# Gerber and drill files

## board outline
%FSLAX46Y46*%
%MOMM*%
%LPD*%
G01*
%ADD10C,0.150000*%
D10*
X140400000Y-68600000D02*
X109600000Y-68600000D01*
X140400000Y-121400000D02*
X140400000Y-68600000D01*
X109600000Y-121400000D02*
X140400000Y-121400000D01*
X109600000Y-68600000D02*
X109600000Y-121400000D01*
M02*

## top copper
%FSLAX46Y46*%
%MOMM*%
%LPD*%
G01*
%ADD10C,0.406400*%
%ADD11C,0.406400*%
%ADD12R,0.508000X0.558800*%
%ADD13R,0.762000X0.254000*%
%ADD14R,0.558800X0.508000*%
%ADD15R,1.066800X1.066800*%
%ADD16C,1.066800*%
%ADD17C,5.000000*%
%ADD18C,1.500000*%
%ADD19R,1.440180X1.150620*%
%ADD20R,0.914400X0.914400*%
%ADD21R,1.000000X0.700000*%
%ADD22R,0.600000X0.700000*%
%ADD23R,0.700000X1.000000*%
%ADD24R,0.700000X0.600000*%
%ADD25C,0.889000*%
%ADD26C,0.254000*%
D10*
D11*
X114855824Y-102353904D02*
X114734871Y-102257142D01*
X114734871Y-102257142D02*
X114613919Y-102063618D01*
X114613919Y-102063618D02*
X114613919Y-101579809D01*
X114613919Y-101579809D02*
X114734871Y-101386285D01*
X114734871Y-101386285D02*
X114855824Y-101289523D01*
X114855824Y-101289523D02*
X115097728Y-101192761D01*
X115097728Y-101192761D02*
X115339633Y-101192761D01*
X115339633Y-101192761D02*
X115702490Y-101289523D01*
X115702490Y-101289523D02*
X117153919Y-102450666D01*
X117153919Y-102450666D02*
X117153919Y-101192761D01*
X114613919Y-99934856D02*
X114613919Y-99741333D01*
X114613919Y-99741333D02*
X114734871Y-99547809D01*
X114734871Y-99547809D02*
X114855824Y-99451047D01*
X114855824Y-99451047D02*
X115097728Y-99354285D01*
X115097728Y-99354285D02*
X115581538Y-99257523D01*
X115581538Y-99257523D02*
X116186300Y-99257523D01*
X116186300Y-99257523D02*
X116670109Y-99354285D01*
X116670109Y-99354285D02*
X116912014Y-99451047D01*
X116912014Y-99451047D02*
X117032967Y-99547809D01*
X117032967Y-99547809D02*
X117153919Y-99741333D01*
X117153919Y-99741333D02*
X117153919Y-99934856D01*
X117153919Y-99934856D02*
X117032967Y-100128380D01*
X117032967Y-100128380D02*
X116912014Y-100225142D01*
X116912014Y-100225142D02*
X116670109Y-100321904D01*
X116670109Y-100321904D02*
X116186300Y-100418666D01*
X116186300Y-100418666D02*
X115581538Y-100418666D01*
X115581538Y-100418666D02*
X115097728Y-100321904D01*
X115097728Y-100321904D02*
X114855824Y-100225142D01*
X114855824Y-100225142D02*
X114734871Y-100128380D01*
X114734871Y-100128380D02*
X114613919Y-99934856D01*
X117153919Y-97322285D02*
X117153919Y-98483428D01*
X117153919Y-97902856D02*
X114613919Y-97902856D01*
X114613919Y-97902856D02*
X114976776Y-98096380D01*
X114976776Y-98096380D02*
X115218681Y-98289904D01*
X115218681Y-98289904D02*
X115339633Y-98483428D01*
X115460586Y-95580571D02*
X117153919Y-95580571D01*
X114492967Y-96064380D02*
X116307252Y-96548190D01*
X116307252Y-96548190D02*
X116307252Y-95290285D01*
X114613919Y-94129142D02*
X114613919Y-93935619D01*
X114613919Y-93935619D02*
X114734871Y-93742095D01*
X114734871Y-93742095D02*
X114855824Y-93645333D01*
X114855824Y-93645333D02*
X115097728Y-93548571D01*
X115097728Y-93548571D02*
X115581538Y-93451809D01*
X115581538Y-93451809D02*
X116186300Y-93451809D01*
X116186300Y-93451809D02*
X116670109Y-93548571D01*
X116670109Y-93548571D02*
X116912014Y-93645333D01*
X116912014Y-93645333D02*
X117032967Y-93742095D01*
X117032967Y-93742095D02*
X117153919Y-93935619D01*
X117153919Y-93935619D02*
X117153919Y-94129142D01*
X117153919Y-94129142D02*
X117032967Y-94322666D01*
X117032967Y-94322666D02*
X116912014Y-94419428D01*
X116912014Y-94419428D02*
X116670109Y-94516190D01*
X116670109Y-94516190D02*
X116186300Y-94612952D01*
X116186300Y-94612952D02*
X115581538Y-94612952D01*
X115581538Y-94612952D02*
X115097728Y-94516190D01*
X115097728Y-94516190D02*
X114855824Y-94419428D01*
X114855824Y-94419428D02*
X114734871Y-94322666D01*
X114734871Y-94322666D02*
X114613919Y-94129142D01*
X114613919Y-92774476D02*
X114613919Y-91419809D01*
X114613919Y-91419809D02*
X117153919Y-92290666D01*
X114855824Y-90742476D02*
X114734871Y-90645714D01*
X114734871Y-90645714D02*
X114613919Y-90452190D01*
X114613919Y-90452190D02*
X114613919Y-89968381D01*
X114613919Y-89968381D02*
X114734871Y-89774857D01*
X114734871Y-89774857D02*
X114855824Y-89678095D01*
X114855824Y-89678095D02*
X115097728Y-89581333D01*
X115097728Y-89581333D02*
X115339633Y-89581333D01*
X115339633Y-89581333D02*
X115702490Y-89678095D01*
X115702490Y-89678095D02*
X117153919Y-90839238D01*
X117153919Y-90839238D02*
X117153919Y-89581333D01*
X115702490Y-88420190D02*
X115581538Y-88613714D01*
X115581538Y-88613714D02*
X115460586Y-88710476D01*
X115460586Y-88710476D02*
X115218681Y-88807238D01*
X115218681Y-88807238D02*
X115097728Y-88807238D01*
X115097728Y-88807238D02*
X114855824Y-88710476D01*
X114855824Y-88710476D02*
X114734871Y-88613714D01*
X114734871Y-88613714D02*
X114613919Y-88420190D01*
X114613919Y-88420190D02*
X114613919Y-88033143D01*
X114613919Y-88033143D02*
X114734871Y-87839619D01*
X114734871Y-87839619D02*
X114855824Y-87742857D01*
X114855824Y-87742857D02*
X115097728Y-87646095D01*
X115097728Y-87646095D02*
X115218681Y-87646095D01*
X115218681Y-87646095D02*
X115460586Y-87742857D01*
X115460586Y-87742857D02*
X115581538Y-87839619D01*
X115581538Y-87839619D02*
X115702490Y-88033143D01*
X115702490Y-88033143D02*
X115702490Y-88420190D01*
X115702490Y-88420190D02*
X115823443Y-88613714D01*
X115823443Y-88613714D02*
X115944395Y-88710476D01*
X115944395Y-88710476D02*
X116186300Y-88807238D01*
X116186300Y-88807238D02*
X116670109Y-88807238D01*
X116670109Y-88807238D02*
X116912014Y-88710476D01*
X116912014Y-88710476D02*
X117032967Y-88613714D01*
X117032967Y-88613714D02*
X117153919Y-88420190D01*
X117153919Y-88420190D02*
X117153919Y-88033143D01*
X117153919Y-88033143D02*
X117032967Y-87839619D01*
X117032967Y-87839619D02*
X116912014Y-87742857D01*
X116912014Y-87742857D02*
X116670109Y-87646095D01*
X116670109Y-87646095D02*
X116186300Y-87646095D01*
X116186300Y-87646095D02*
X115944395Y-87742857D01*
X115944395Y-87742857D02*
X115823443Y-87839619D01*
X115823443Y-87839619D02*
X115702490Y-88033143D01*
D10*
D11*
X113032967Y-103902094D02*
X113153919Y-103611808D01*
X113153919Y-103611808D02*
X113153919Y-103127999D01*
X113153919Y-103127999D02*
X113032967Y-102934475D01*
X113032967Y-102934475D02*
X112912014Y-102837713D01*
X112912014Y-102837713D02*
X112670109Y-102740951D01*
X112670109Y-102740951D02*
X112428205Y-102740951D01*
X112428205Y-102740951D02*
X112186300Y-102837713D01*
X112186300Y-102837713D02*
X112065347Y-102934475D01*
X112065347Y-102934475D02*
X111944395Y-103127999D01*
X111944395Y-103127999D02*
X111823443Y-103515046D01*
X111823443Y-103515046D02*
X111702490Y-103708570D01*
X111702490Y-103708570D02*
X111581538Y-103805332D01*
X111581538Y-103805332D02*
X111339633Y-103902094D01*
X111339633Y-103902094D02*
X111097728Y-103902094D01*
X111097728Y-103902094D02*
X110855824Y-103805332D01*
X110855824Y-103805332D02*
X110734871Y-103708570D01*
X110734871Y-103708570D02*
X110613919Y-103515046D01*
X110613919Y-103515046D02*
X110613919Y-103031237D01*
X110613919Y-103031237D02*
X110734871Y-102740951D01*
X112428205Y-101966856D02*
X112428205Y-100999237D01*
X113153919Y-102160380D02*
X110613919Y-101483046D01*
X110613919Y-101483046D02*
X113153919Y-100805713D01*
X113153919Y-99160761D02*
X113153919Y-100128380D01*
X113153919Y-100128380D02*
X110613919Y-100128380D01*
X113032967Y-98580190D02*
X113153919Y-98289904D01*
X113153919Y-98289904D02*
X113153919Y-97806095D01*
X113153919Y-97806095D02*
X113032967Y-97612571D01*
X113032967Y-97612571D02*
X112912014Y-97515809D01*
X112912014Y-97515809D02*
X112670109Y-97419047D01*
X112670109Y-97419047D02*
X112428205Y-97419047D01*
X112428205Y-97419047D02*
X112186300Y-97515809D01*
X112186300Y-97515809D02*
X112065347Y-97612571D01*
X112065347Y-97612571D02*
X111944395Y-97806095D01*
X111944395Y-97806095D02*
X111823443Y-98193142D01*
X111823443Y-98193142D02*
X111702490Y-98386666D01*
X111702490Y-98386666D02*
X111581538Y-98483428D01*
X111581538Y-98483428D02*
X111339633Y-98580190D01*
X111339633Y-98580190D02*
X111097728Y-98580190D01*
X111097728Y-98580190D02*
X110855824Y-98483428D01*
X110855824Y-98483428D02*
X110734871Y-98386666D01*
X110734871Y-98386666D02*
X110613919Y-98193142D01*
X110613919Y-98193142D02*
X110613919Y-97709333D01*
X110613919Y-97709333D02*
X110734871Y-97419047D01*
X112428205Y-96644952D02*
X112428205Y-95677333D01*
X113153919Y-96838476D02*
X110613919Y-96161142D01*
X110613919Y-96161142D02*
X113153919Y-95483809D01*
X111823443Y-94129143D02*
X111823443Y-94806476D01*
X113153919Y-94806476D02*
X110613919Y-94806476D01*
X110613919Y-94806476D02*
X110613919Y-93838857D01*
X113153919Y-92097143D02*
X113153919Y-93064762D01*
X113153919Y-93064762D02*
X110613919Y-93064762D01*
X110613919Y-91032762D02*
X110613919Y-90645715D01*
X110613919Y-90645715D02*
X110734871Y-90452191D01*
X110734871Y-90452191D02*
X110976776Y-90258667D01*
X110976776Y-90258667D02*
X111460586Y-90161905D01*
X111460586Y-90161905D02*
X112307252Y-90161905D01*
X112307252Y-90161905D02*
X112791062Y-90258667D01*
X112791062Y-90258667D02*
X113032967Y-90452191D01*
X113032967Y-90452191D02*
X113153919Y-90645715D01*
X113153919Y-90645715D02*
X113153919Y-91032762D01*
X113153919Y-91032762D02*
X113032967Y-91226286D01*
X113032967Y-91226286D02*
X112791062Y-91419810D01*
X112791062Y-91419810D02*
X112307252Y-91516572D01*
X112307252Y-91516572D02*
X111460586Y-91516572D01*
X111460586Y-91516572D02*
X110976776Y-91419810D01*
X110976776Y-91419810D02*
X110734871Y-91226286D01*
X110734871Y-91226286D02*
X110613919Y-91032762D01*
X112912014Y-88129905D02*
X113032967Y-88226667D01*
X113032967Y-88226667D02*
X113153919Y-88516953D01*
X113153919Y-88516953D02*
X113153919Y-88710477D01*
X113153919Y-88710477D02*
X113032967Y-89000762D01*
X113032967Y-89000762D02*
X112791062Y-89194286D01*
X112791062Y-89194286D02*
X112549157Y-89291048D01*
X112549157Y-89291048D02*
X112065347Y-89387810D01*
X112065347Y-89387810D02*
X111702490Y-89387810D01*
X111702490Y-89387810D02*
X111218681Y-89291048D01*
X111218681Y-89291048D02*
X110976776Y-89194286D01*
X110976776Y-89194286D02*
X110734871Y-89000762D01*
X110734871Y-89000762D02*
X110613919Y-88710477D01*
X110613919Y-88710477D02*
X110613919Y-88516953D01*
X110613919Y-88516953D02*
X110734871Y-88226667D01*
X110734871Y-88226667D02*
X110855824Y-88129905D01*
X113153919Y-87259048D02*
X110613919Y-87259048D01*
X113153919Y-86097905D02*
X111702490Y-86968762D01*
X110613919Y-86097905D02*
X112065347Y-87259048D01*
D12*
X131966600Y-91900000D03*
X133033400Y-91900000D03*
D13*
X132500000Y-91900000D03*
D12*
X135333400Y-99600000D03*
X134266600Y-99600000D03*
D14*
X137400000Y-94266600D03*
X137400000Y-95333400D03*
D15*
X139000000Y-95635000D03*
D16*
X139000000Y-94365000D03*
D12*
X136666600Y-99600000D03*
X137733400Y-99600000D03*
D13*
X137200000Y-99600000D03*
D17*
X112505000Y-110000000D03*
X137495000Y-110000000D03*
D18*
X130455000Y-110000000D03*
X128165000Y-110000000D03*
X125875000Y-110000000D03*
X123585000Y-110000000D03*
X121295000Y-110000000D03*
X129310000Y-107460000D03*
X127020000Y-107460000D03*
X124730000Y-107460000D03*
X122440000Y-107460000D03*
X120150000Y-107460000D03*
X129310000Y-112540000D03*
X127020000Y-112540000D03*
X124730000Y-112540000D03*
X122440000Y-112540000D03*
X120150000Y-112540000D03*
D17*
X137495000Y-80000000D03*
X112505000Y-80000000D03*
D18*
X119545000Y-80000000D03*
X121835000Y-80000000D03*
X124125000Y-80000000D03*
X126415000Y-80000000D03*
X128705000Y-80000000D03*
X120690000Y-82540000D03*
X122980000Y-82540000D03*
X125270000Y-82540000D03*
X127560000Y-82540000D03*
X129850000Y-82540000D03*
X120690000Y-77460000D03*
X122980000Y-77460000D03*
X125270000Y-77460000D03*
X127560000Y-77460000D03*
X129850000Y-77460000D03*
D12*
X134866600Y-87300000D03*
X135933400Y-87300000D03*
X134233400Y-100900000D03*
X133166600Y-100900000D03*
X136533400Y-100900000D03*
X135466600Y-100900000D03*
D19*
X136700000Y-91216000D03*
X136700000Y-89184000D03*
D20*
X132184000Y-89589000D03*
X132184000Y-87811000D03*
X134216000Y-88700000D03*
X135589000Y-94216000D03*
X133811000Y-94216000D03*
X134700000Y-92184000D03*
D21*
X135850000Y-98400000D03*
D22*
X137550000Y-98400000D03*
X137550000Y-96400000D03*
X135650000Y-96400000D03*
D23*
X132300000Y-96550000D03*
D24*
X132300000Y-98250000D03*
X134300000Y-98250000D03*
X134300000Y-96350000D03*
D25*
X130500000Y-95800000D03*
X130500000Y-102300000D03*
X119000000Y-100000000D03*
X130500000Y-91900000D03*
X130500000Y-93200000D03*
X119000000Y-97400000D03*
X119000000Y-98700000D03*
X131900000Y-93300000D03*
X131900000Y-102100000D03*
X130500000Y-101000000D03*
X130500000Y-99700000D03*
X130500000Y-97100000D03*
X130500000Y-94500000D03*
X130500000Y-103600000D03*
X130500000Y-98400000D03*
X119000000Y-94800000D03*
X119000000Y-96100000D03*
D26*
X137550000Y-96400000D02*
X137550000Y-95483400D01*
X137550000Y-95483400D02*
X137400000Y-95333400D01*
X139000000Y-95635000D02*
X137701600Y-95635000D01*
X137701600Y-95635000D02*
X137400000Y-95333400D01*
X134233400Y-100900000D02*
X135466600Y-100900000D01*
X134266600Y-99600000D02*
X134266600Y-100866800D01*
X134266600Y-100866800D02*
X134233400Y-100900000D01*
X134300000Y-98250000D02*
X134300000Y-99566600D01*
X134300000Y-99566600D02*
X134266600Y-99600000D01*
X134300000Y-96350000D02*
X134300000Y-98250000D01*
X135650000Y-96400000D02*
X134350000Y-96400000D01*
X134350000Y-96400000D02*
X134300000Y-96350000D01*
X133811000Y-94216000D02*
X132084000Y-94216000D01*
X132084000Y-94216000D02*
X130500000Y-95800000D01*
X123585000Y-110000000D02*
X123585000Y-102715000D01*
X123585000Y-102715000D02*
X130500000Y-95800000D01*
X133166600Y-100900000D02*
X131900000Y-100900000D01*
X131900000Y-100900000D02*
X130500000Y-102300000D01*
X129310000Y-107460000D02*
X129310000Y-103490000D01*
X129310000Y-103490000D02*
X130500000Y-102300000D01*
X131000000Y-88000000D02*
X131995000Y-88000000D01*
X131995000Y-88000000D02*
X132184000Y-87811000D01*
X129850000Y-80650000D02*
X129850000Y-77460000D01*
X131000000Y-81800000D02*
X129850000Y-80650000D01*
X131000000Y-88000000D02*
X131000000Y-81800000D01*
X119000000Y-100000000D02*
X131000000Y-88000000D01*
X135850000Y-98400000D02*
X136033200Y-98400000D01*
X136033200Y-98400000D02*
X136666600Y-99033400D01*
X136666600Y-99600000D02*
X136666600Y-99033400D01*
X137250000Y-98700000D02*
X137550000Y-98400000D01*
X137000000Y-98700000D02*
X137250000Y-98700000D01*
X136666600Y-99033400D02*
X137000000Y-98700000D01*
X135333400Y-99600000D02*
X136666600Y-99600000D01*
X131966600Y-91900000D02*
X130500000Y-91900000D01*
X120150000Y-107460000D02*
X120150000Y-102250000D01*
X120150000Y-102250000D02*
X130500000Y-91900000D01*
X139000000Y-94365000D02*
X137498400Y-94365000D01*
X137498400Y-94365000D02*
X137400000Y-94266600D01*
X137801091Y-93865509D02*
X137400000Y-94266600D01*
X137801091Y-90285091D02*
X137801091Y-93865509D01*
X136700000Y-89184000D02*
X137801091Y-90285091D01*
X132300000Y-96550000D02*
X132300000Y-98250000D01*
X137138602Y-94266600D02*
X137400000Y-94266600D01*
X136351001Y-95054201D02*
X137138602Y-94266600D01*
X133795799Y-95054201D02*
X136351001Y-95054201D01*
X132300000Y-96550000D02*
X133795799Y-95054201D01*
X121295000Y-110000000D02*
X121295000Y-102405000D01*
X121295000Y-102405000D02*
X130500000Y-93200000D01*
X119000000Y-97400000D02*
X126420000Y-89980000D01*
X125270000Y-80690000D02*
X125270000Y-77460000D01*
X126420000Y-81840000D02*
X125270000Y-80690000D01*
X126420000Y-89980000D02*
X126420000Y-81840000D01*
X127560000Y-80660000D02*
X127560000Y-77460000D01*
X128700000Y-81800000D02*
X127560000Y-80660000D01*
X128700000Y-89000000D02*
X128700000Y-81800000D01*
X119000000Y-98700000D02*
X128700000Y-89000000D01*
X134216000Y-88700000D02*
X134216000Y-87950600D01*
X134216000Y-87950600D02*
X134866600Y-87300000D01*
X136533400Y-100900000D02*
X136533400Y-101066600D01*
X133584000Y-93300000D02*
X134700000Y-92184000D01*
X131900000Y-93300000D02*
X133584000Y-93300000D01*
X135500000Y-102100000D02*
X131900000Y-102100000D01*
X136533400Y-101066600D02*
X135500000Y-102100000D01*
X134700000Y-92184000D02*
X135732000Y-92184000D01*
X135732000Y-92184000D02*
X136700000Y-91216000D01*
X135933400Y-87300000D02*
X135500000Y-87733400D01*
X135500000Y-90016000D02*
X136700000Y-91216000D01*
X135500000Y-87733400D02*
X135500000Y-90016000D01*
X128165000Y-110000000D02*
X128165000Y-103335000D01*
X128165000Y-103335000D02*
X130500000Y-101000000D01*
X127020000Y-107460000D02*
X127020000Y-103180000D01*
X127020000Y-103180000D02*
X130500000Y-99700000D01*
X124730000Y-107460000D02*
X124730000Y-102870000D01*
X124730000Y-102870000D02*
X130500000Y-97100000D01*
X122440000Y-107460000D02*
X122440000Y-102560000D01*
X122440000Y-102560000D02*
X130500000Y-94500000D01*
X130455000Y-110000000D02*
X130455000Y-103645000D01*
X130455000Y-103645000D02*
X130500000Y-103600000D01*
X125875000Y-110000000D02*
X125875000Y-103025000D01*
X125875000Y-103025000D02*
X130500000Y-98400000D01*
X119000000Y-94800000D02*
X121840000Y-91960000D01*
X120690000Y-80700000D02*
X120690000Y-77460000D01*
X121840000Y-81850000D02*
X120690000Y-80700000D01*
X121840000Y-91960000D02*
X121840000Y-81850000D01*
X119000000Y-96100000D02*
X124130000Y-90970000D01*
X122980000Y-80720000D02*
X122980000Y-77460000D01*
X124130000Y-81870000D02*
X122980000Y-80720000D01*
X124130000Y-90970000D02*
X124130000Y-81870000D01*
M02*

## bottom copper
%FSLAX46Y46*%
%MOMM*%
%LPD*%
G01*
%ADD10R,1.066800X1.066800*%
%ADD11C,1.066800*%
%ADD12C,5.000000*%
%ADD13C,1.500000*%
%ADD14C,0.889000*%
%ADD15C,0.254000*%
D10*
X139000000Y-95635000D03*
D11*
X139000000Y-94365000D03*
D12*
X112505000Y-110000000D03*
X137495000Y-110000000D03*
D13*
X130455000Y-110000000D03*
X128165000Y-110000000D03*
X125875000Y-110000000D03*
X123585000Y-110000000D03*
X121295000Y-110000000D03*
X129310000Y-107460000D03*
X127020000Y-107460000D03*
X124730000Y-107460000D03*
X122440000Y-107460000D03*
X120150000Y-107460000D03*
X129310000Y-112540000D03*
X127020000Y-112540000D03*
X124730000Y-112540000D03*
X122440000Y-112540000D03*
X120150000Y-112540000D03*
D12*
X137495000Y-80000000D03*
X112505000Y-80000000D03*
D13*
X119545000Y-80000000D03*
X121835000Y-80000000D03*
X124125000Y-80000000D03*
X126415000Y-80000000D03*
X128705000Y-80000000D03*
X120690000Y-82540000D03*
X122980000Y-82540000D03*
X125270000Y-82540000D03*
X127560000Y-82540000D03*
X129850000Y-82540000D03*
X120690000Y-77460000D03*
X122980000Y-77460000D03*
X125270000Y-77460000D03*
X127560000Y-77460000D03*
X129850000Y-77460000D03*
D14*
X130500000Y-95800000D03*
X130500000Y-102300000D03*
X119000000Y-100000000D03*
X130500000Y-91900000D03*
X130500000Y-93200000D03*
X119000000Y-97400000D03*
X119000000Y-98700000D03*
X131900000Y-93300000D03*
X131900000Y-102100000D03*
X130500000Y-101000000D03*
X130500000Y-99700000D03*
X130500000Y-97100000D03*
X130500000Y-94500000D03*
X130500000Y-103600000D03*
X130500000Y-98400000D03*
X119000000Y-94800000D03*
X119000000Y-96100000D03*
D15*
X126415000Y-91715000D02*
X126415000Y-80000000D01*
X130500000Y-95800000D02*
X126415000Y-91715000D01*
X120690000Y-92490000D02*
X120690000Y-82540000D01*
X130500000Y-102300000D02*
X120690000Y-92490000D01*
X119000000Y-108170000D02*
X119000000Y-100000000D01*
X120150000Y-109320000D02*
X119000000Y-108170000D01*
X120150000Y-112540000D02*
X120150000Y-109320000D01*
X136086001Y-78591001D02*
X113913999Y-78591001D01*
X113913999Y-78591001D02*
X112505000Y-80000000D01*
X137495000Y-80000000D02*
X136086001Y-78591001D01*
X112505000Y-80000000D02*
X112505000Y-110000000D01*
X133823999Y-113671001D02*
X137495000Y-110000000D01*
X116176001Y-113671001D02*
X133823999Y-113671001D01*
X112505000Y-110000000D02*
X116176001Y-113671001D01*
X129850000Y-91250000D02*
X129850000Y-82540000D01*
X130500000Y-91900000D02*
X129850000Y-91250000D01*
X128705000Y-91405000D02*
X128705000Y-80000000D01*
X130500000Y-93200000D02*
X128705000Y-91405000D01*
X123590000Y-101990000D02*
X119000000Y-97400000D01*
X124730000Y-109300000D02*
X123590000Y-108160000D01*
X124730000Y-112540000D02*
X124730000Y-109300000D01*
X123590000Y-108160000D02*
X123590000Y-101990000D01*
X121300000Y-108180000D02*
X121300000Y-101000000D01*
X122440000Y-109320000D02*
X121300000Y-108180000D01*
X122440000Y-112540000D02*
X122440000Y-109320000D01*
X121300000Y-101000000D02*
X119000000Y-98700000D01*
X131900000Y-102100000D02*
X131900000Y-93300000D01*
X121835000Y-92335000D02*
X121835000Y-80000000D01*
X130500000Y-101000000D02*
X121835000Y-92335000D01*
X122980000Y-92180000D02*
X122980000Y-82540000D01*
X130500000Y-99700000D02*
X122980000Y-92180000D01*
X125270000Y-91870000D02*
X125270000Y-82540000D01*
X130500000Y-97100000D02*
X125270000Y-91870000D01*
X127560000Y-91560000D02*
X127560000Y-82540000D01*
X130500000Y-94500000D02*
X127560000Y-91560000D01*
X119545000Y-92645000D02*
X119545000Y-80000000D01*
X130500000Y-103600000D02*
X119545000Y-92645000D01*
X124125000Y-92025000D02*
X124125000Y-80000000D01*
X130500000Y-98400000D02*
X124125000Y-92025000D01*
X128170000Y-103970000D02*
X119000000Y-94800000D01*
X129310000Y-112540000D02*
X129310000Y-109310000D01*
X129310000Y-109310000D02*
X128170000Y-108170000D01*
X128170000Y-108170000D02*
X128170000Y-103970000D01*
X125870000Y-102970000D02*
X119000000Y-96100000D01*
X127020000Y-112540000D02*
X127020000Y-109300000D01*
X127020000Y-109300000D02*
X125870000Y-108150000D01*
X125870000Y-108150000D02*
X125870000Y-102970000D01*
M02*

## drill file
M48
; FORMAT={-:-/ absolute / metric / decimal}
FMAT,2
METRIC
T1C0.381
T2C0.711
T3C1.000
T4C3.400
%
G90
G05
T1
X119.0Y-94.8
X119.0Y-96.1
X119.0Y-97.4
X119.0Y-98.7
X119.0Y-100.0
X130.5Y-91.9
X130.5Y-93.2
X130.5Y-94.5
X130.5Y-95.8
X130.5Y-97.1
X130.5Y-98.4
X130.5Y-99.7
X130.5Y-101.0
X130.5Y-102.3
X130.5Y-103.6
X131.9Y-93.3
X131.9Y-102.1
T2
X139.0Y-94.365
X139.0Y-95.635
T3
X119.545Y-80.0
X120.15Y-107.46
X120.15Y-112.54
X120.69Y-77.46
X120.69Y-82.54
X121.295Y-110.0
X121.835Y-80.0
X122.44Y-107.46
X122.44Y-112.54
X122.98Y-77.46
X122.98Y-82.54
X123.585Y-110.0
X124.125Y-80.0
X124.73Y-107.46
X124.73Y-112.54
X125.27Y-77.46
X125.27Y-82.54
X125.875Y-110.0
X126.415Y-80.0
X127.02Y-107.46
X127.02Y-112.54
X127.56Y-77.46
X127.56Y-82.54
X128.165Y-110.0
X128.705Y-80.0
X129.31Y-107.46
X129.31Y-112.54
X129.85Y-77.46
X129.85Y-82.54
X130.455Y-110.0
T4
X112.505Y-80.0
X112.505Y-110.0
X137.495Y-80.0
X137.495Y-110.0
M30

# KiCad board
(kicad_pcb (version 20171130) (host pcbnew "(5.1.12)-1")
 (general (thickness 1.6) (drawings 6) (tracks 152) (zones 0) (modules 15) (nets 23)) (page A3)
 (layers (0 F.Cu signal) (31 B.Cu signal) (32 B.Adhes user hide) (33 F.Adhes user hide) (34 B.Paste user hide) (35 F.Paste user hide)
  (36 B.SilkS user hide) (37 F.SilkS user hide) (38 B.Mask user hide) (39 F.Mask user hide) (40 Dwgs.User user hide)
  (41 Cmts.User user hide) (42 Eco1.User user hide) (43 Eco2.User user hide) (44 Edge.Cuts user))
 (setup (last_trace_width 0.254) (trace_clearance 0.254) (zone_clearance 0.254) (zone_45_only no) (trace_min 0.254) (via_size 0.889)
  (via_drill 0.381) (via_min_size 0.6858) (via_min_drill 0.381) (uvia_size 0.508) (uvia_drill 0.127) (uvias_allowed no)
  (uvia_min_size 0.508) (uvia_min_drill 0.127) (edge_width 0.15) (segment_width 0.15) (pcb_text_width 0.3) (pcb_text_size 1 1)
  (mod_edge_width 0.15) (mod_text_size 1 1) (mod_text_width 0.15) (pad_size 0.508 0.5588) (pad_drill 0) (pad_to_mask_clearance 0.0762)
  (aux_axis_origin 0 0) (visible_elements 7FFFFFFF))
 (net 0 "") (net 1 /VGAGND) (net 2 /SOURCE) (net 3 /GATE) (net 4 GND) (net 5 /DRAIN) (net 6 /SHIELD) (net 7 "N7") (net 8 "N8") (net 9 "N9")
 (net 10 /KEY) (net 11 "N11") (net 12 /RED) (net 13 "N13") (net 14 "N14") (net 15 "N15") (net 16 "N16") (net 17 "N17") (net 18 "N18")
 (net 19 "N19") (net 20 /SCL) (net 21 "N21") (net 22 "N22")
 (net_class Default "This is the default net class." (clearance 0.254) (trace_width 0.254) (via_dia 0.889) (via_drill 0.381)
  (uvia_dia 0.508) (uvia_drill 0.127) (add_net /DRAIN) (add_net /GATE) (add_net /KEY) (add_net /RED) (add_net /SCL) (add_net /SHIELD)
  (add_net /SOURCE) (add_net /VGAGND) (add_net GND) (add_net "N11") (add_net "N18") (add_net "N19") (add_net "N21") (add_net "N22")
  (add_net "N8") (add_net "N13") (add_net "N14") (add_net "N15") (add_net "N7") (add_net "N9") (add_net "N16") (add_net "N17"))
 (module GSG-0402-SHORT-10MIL (layer F.Cu) (at 132.5 91.9 180) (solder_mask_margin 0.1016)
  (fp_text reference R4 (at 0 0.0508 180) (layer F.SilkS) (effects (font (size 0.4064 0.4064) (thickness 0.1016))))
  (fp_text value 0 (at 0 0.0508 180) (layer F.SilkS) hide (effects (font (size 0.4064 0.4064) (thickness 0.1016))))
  (pad 2 smd rect (at 0.5334 0 180) (size 0.508 0.5588) (layers F.Cu F.Mask) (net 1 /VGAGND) (solder_mask_margin 0.1016))
  (pad 1 smd rect (at -0.5334 0 180) (size 0.508 0.5588) (layers F.Cu F.Mask) (die_length -1518.485687) (solder_mask_margin 0.1016))
  (pad "" smd rect (at 0 0 180) (size 0.762 0.254) (layers F.Cu F.Mask)))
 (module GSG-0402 (layer F.Cu) (at 134.8 99.6) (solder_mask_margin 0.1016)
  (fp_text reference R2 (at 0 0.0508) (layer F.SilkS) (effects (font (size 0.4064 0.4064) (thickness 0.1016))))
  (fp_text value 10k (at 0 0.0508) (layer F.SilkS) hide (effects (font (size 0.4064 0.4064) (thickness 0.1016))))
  (pad 2 smd rect (at 0.5334 0) (size 0.508 0.5588) (layers F.Cu F.Paste F.Mask) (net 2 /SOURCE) (solder_mask_margin 0.1016))
  (pad 1 smd rect (at -0.5334 0) (size 0.508 0.5588) (layers F.Cu F.Paste F.Mask) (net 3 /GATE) (die_length -1518.485687)
   (solder_mask_margin 0.1016)))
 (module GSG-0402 (layer F.Cu) (at 137.4 94.8 90) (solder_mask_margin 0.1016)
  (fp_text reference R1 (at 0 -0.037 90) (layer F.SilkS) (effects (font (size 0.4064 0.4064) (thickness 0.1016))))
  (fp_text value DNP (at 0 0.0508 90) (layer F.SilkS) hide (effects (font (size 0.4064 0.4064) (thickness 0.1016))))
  (pad 2 smd rect (at 0.5334 0 90) (size 0.508 0.5588) (layers F.Cu F.Paste F.Mask) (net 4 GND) (solder_mask_margin 0.1016))
  (pad 1 smd rect (at -0.5334 0 90) (size 0.508 0.5588) (layers F.Cu F.Paste F.Mask) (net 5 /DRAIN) (die_length -1518.485687)
   (solder_mask_margin 0.1016)))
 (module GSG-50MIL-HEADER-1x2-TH (layer F.Cu) (at 139 95 90)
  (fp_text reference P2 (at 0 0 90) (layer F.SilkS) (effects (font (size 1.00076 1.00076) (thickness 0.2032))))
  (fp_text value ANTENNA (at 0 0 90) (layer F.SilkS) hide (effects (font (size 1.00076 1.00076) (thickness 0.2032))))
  (pad 1 thru_hole rect (at -0.635 0 90) (size 1.0668 1.0668) (drill 0.7112) (layers *.Cu *.Mask) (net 5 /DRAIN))
  (pad 2 thru_hole circle (at 0.635 0 90) (size 1.0668 1.0668) (drill 0.7112) (layers *.Cu *.Mask) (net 4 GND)))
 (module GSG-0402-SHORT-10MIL (layer F.Cu) (at 137.2 99.6 180) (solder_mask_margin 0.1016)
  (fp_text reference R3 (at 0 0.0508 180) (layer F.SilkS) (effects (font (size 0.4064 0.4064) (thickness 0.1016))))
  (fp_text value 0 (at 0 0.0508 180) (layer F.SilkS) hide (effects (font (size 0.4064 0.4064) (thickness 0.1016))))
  (pad 2 smd rect (at 0.5334 0 180) (size 0.508 0.5588) (layers F.Cu F.Mask) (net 2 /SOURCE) (solder_mask_margin 0.1016))
  (pad 1 smd rect (at -0.5334 0 180) (size 0.508 0.5588) (layers F.Cu F.Mask) (die_length -1518.485687) (solder_mask_margin 0.1016))
  (pad "" smd rect (at 0 0 180) (size 0.762 0.254) (layers F.Cu F.Mask)))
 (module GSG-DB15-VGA (layer F.Cu) (at 125 110)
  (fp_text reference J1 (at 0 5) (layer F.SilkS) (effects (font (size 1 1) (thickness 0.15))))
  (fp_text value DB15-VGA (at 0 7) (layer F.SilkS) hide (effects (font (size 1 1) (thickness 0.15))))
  (pad 0 thru_hole circle (at -12.495 0) (size 5 5) (drill 3.4) (layers *.Cu *.Mask) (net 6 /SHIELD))
  (pad 0 thru_hole circle (at 12.495 0) (size 5 5) (drill 3.4) (layers *.Cu *.Mask) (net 6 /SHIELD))
  (pad 6 thru_hole circle (at 5.455 0) (size 1.5 1.5) (drill 1) (layers *.Cu *.Mask) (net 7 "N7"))
  (pad 7 thru_hole circle (at 3.165 0) (size 1.5 1.5) (drill 1) (layers *.Cu *.Mask) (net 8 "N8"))
  (pad 8 thru_hole circle (at 0.875 0) (size 1.5 1.5) (drill 1) (layers *.Cu *.Mask) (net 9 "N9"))
  (pad 9 thru_hole circle (at -1.415 0) (size 1.5 1.5) (drill 1) (layers *.Cu *.Mask) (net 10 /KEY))
  (pad 10 thru_hole circle (at -3.705 0) (size 1.5 1.5) (drill 1) (layers *.Cu *.Mask) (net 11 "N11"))
  (pad 1 thru_hole circle (at 4.31 -2.54) (size 1.5 1.5) (drill 1) (layers *.Cu *.Mask) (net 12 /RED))
  (pad 2 thru_hole circle (at 2.02 -2.54) (size 1.5 1.5) (drill 1) (layers *.Cu *.Mask) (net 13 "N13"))
  (pad 3 thru_hole circle (at -0.27 -2.54) (size 1.5 1.5) (drill 1) (layers *.Cu *.Mask) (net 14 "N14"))
  (pad 4 thru_hole circle (at -2.56 -2.54) (size 1.5 1.5) (drill 1) (layers *.Cu *.Mask) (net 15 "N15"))
  (pad 5 thru_hole circle (at -4.85 -2.54) (size 1.5 1.5) (drill 1) (layers *.Cu *.Mask) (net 1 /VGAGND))
  (pad 11 thru_hole circle (at 4.31 2.54) (size 1.5 1.5) (drill 1) (layers *.Cu *.Mask) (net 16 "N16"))
  (pad 12 thru_hole circle (at 2.02 2.54) (size 1.5 1.5) (drill 1) (layers *.Cu *.Mask) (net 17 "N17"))
  (pad 13 thru_hole circle (at -0.27 2.54) (size 1.5 1.5) (drill 1) (layers *.Cu *.Mask) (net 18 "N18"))
  (pad 14 thru_hole circle (at -2.56 2.54) (size 1.5 1.5) (drill 1) (layers *.Cu *.Mask) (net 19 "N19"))
  (pad 15 thru_hole circle (at -4.85 2.54) (size 1.5 1.5) (drill 1) (layers *.Cu *.Mask) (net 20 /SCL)))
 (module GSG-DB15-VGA (layer F.Cu) (at 125 80 180)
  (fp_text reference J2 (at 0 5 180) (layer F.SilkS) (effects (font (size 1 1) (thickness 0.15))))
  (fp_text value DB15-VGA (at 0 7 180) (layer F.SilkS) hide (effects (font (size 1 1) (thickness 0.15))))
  (pad 0 thru_hole circle (at -12.495 0 180) (size 5 5) (drill 3.4) (layers *.Cu *.Mask) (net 6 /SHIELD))
  (pad 0 thru_hole circle (at 12.495 0 180) (size 5 5) (drill 3.4) (layers *.Cu *.Mask) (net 6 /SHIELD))
  (pad 6 thru_hole circle (at 5.455 0 180) (size 1.5 1.5) (drill 1) (layers *.Cu *.Mask) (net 7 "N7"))
  (pad 7 thru_hole circle (at 3.165 0 180) (size 1.5 1.5) (drill 1) (layers *.Cu *.Mask) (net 8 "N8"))
  (pad 8 thru_hole circle (at 0.875 0 180) (size 1.5 1.5) (drill 1) (layers *.Cu *.Mask) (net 9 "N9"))
  (pad 9 thru_hole circle (at -1.415 0 180) (size 1.5 1.5) (drill 1) (layers *.Cu *.Mask) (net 10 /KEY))
  (pad 10 thru_hole circle (at -3.705 0 180) (size 1.5 1.5) (drill 1) (layers *.Cu *.Mask) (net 11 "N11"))
  (pad 1 thru_hole circle (at 4.31 -2.54 180) (size 1.5 1.5) (drill 1) (layers *.Cu *.Mask) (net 12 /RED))
  (pad 2 thru_hole circle (at 2.02 -2.54 180) (size 1.5 1.5) (drill 1) (layers *.Cu *.Mask) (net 13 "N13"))
  (pad 3 thru_hole circle (at -0.27 -2.54 180) (size 1.5 1.5) (drill 1) (layers *.Cu *.Mask) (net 14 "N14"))
  (pad 4 thru_hole circle (at -2.56 -2.54 180) (size 1.5 1.5) (drill 1) (layers *.Cu *.Mask) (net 15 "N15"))
  (pad 5 thru_hole circle (at -4.85 -2.54 180) (size 1.5 1.5) (drill 1) (layers *.Cu *.Mask) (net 1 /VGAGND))
  (pad 11 thru_hole circle (at 4.31 2.54 180) (size 1.5 1.5) (drill 1) (layers *.Cu *.Mask) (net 16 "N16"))
  (pad 12 thru_hole circle (at 2.02 2.54 180) (size 1.5 1.5) (drill 1) (layers *.Cu *.Mask) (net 17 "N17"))
  (pad 13 thru_hole circle (at -0.27 2.54 180) (size 1.5 1.5) (drill 1) (layers *.Cu *.Mask) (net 18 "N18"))
  (pad 14 thru_hole circle (at -2.56 2.54 180) (size 1.5 1.5) (drill 1) (layers *.Cu *.Mask) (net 19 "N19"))
  (pad 15 thru_hole circle (at -4.85 2.54 180) (size 1.5 1.5) (drill 1) (layers *.Cu *.Mask) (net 20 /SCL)))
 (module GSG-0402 (layer F.Cu) (at 135.4 87.3 180) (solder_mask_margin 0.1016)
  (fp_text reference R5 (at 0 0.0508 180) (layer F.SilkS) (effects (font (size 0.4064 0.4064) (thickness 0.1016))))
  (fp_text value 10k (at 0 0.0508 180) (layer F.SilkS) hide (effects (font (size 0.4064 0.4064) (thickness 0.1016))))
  (pad 2 smd rect (at 0.5334 0 180) (size 0.508 0.5588) (layers F.Cu F.Paste F.Mask) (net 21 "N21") (solder_mask_margin 0.1016))
  (pad 1 smd rect (at -0.5334 0 180) (size 0.508 0.5588) (layers F.Cu F.Paste F.Mask) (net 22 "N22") (die_length -1518.485687)
   (solder_mask_margin 0.1016)))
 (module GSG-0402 (layer F.Cu) (at 133.7 100.9) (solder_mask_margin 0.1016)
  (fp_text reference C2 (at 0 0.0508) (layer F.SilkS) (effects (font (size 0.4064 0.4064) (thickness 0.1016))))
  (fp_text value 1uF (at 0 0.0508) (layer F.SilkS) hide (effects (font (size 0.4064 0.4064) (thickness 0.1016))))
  (pad 2 smd rect (at 0.5334 0) (size 0.508 0.5588) (layers F.Cu F.Paste F.Mask) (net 3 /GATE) (solder_mask_margin 0.1016))
  (pad 1 smd rect (at -0.5334 0) (size 0.508 0.5588) (layers F.Cu F.Paste F.Mask) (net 12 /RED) (die_length -1518.485687)
   (solder_mask_margin 0.1016)))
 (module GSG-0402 (layer F.Cu) (at 136 100.9) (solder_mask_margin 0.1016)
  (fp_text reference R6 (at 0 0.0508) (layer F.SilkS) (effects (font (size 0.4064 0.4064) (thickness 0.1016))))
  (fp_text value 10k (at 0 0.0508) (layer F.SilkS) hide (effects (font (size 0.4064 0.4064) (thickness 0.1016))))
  (pad 2 smd rect (at 0.5334 0) (size 0.508 0.5588) (layers F.Cu F.Paste F.Mask) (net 22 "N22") (solder_mask_margin 0.1016))
  (pad 1 smd rect (at -0.5334 0) (size 0.508 0.5588) (layers F.Cu F.Paste F.Mask) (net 3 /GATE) (die_length -1518.485687)
   (solder_mask_margin 0.1016)))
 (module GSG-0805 (layer F.Cu) (at 136.7 90.2 270) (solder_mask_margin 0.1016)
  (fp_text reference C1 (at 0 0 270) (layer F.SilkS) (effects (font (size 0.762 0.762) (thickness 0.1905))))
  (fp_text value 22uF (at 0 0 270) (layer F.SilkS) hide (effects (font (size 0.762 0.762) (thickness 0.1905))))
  (pad 2 smd rect (at 1.016 0 270) (size 1.15062 1.44018) (layers F.Cu F.Paste F.Mask) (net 22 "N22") (die_length 0.08128)
   (solder_mask_margin 0.1016) (clearance 0.1778))
  (pad 1 smd rect (at -1.016 0 270) (size 1.15062 1.44018) (layers F.Cu F.Paste F.Mask) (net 4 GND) (die_length -1518.485687)
   (solder_mask_margin 0.1016) (clearance 0.1778)))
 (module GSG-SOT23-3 (layer F.Cu) (at 133.2 88.7 90)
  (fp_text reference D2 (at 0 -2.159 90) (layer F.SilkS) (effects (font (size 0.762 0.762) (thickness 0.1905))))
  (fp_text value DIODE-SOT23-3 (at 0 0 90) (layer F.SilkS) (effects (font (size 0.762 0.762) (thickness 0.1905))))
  (pad 2 smd rect (at -0.889 -1.016 90) (size 0.9144 0.9144) (layers F.Cu F.Paste F.Mask) (die_length 0.00762))
  (pad 1 smd rect (at 0.889 -1.016 90) (size 0.9144 0.9144) (layers F.Cu F.Paste F.Mask) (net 20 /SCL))
  (pad 3 smd rect (at 0 1.016 90) (size 0.9144 0.9144) (layers F.Cu F.Paste F.Mask) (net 21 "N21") (die_length 0.28194)))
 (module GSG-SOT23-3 (layer F.Cu) (at 134.7 93.2 180)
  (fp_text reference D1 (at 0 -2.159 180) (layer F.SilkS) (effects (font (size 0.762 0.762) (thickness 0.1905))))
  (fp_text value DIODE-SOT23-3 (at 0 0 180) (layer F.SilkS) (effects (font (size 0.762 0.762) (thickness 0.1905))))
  (pad 2 smd rect (at -0.889 -1.016 180) (size 0.9144 0.9144) (layers F.Cu F.Paste F.Mask) (die_length 0.00762))
  (pad 1 smd rect (at 0.889 -1.016 180) (size 0.9144 0.9144) (layers F.Cu F.Paste F.Mask) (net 10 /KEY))
  (pad 3 smd rect (at 0 1.016 180) (size 0.9144 0.9144) (layers F.Cu F.Paste F.Mask) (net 22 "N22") (die_length 0.28194)))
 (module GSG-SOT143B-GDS (layer F.Cu) (at 136.6 97.4)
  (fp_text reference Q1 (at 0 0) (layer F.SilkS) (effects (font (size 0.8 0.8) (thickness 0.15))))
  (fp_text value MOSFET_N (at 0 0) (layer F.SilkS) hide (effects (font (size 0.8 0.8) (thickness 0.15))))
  (pad B smd rect (at -0.75 1) (size 1 0.7) (layers F.Cu F.Paste F.Mask) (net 2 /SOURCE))
  (pad S smd rect (at 0.95 1) (size 0.6 0.7) (layers F.Cu F.Paste F.Mask) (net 2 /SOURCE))
  (pad D smd rect (at 0.95 -1) (size 0.6 0.7) (layers F.Cu F.Paste F.Mask) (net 5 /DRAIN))
  (pad G smd rect (at -0.95 -1) (size 0.6 0.7) (layers F.Cu F.Paste F.Mask) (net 3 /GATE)))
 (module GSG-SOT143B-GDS (layer F.Cu) (at 133.3 97.3 270)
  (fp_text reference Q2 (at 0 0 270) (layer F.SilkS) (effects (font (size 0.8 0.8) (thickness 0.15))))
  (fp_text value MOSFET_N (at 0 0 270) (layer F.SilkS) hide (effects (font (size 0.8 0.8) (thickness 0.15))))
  (pad B smd rect (at -0.75 1 270) (size 1 0.7) (layers F.Cu F.Paste F.Mask) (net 4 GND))
  (pad S smd rect (at 0.95 1 270) (size 0.6 0.7) (layers F.Cu F.Paste F.Mask) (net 4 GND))
  (pad D smd rect (at 0.95 -1 270) (size 0.6 0.7) (layers F.Cu F.Paste F.Mask) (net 3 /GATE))
  (pad G smd rect (at -0.95 -1 270) (size 0.6 0.7) (layers F.Cu F.Paste F.Mask) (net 3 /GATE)))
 (gr_line (start 140.4 68.6) (end 109.6 68.6) (angle 90) (layer Edge.Cuts) (width 0.15))
 (gr_line (start 140.4 121.4) (end 140.4 68.6) (angle 90) (layer Edge.Cuts) (width 0.15))
 (gr_line (start 109.6 121.4) (end 140.4 121.4) (angle 90) (layer Edge.Cuts) (width 0.15))
 (gr_line (start 109.6 68.6) (end 109.6 121.4) (angle 90) (layer Edge.Cuts) (width 0.15))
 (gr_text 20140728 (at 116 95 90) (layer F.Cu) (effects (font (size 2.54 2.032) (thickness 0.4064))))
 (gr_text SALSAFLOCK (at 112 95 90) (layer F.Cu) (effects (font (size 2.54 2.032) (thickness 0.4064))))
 (segment (start 137.55 96.4) (end 137.55 95.4834) (width 0.254) (layer F.Cu) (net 5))
 (segment (start 137.55 95.4834) (end 137.4 95.3334) (width 0.254) (layer F.Cu) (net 5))
 (segment (start 139 95.635) (end 137.7016 95.635) (width 0.254) (layer F.Cu) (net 5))
 (segment (start 137.7016 95.635) (end 137.4 95.3334) (width 0.254) (layer F.Cu) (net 5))
 (segment (start 134.2334 100.9) (end 135.4666 100.9) (width 0.254) (layer F.Cu) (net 3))
 (segment (start 134.2666 99.6) (end 134.2666 100.8668) (width 0.254) (layer F.Cu) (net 3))
 (segment (start 134.2666 100.8668) (end 134.2334 100.9) (width 0.254) (layer F.Cu) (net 3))
 (segment (start 134.3 98.25) (end 134.3 99.5666) (width 0.254) (layer F.Cu) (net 3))
 (segment (start 134.3 99.5666) (end 134.2666 99.6) (width 0.254) (layer F.Cu) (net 3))
 (segment (start 134.3 96.35) (end 134.3 98.25) (width 0.254) (layer F.Cu) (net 3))
 (segment (start 135.65 96.4) (end 134.35 96.4) (width 0.254) (layer F.Cu) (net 3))
 (segment (start 134.35 96.4) (end 134.3 96.35) (width 0.254) (layer F.Cu) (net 3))
 (segment (start 133.811 94.216) (end 132.084 94.216) (width 0.254) (layer F.Cu) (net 10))
 (segment (start 132.084 94.216) (end 130.5 95.8) (width 0.254) (layer F.Cu) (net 10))
 (segment (start 123.585 110) (end 123.585 102.715) (width 0.254) (layer F.Cu) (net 10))
 (segment (start 126.415 91.715) (end 126.415 80) (width 0.254) (layer B.Cu) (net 10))
 (segment (start 130.5 95.8) (end 126.415 91.715) (width 0.254) (layer B.Cu) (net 10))
 (via (at 130.5 95.8) (size 0.889) (layers F.Cu B.Cu) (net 10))
 (segment (start 123.585 102.715) (end 130.5 95.8) (width 0.254) (layer F.Cu) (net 10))
 (segment (start 133.1666 100.9) (end 131.9 100.9) (width 0.254) (layer F.Cu) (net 12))
 (segment (start 131.9 100.9) (end 130.5 102.3) (width 0.254) (layer F.Cu) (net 12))
 (segment (start 129.31 107.46) (end 129.31 103.49) (width 0.254) (layer F.Cu) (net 12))
 (segment (start 120.69 92.49) (end 120.69 82.54) (width 0.254) (layer B.Cu) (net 12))
 (segment (start 130.5 102.3) (end 120.69 92.49) (width 0.254) (layer B.Cu) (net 12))
 (via (at 130.5 102.3) (size 0.889) (layers F.Cu B.Cu) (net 12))
 (segment (start 129.31 103.49) (end 130.5 102.3) (width 0.254) (layer F.Cu) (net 12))
 (segment (start 131 88) (end 131.995 88) (width 0.254) (layer F.Cu) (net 20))
 (segment (start 131.995 88) (end 132.184 87.811) (width 0.254) (layer F.Cu) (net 20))
 (segment (start 119 108.17) (end 119 100) (width 0.254) (layer B.Cu) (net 20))
 (segment (start 120.15 109.32) (end 119 108.17) (width 0.254) (layer B.Cu) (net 20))
 (segment (start 120.15 112.54) (end 120.15 109.32) (width 0.254) (layer B.Cu) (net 20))
 (segment (start 129.85 80.65) (end 129.85 77.46) (width 0.254) (layer F.Cu) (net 20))
 (segment (start 131 81.8) (end 129.85 80.65) (width 0.254) (layer F.Cu) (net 20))
 (segment (start 131 88) (end 131 81.8) (width 0.254) (layer F.Cu) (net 20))
 (segment (start 119 100) (end 131 88) (width 0.254) (layer F.Cu) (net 20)) (via (at 119 100) (size 0.889) (layers F.Cu B.Cu) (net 20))
 (segment (start 136.086001 78.591001) (end 113.913999 78.591001) (width 0.254) (layer B.Cu) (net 6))
 (segment (start 113.913999 78.591001) (end 112.505 80) (width 0.254) (layer B.Cu) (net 6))
 (segment (start 137.495 80) (end 136.086001 78.591001) (width 0.254) (layer B.Cu) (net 6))
 (segment (start 112.505 80) (end 112.505 110) (width 0.254) (layer B.Cu) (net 6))
 (segment (start 133.823999 113.671001) (end 137.495 110) (width 0.254) (layer B.Cu) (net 6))
 (segment (start 116.176001 113.671001) (end 133.823999 113.671001) (width 0.254) (layer B.Cu) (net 6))
 (segment (start 112.505 110) (end 116.176001 113.671001) (width 0.254) (layer B.Cu) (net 6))
 (segment (start 135.85 98.4) (end 136.0332 98.4) (width 0.254) (layer F.Cu) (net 2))
 (segment (start 136.0332 98.4) (end 136.6666 99.0334) (width 0.254) (layer F.Cu) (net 2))
 (segment (start 136.6666 99.6) (end 136.6666 99.0334) (width 0.254) (layer F.Cu) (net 2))
 (segment (start 137.25 98.7) (end 137.55 98.4) (width 0.254) (layer F.Cu) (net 2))
 (segment (start 137 98.7) (end 137.25 98.7) (width 0.254) (layer F.Cu) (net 2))
 (segment (start 136.6666 99.0334) (end 137 98.7) (width 0.254) (layer F.Cu) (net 2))
 (segment (start 135.3334 99.6) (end 136.6666 99.6) (width 0.254) (layer F.Cu) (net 2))
 (segment (start 131.9666 91.9) (end 130.5 91.9) (width 0.254) (layer F.Cu) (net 1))
 (segment (start 120.15 107.46) (end 120.15 102.25) (width 0.254) (layer F.Cu) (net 1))
 (segment (start 129.85 91.25) (end 129.85 82.54) (width 0.254) (layer B.Cu) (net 1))
 (segment (start 130.5 91.9) (end 129.85 91.25) (width 0.254) (layer B.Cu) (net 1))
 (via (at 130.5 91.9) (size 0.889) (layers F.Cu B.Cu) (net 1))
 (segment (start 120.15 102.25) (end 130.5 91.9) (width 0.254) (layer F.Cu) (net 1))
 (segment (start 139 94.365) (end 137.4984 94.365) (width 0.254) (layer F.Cu) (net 4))
 (segment (start 137.4984 94.365) (end 137.4 94.2666) (width 0.254) (layer F.Cu) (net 4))
 (segment (start 137.801091 93.865509) (end 137.4 94.2666) (width 0.254) (layer F.Cu) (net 4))
 (segment (start 137.801091 90.285091) (end 137.801091 93.865509) (width 0.254) (layer F.Cu) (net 4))
 (segment (start 136.7 89.184) (end 137.801091 90.285091) (width 0.254) (layer F.Cu) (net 4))
 (segment (start 132.3 96.55) (end 132.3 98.25) (width 0.254) (layer F.Cu) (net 4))
 (segment (start 137.138602 94.2666) (end 137.4 94.2666) (width 0.254) (layer F.Cu) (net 4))
 (segment (start 136.351001 95.054201) (end 137.138602 94.2666) (width 0.254) (layer F.Cu) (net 4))
 (segment (start 133.795799 95.054201) (end 136.351001 95.054201) (width 0.254) (layer F.Cu) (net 4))
 (segment (start 132.3 96.55) (end 133.795799 95.054201) (width 0.254) (layer F.Cu) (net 4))
 (segment (start 121.295 110) (end 121.295 102.405) (width 0.254) (layer F.Cu) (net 11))
 (segment (start 128.705 91.405) (end 128.705 80) (width 0.254) (layer B.Cu) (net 11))
 (segment (start 130.5 93.2) (end 128.705 91.405) (width 0.254) (layer B.Cu) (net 11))
 (via (at 130.5 93.2) (size 0.889) (layers F.Cu B.Cu) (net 11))
 (segment (start 121.295 102.405) (end 130.5 93.2) (width 0.254) (layer F.Cu) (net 11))
 (segment (start 119 97.4) (end 126.42 89.98) (width 0.254) (layer F.Cu) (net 18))
 (segment (start 123.59 101.99) (end 119 97.4) (width 0.254) (layer B.Cu) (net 18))
 (via (at 119 97.4) (size 0.889) (layers F.Cu B.Cu) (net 18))
 (segment (start 124.73 109.3) (end 123.59 108.16) (width 0.254) (layer B.Cu) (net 18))
 (segment (start 124.73 112.54) (end 124.73 109.3) (width 0.254) (layer B.Cu) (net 18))
 (segment (start 123.59 108.16) (end 123.59 101.99) (width 0.254) (layer B.Cu) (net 18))
 (segment (start 125.27 80.69) (end 125.27 77.46) (width 0.254) (layer F.Cu) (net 18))
 (segment (start 126.42 81.84) (end 125.27 80.69) (width 0.254) (layer F.Cu) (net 18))
 (segment (start 126.42 89.98) (end 126.42 81.84) (width 0.254) (layer F.Cu) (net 18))
 (segment (start 121.3 108.18) (end 121.3 101) (width 0.254) (layer B.Cu) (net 19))
 (segment (start 122.44 109.32) (end 121.3 108.18) (width 0.254) (layer B.Cu) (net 19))
 (segment (start 122.44 112.54) (end 122.44 109.32) (width 0.254) (layer B.Cu) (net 19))
 (segment (start 127.56 80.66) (end 127.56 77.46) (width 0.254) (layer F.Cu) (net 19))
 (segment (start 128.7 81.8) (end 127.56 80.66) (width 0.254) (layer F.Cu) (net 19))
 (segment (start 128.7 89) (end 128.7 81.8) (width 0.254) (layer F.Cu) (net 19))
 (segment (start 119 98.7) (end 128.7 89) (width 0.254) (layer F.Cu) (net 19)) (via (at 119 98.7) (size 0.889) (layers F.Cu B.Cu) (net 19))
 (segment (start 121.3 101) (end 119 98.7) (width 0.254) (layer B.Cu) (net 19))
 (segment (start 134.216 88.7) (end 134.216 87.9506) (width 0.254) (layer F.Cu) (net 21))
 (segment (start 134.216 87.9506) (end 134.8666 87.3) (width 0.254) (layer F.Cu) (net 21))
 (segment (start 136.5334 100.9) (end 136.5334 101.0666) (width 0.254) (layer F.Cu) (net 22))
 (segment (start 133.584 93.3) (end 134.7 92.184) (width 0.254) (layer F.Cu) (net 22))
 (segment (start 131.9 93.3) (end 133.584 93.3) (width 0.254) (layer F.Cu) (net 22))
 (via (at 131.9 93.3) (size 0.889) (layers F.Cu B.Cu) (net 22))
 (segment (start 131.9 102.1) (end 131.9 93.3) (width 0.254) (layer B.Cu) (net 22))
 (via (at 131.9 102.1) (size 0.889) (layers F.Cu B.Cu) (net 22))
 (segment (start 135.5 102.1) (end 131.9 102.1) (width 0.254) (layer F.Cu) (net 22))
 (segment (start 136.5334 101.0666) (end 135.5 102.1) (width 0.254) (layer F.Cu) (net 22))
 (segment (start 134.7 92.184) (end 135.732 92.184) (width 0.254) (layer F.Cu) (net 22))
 (segment (start 135.732 92.184) (end 136.7 91.216) (width 0.254) (layer F.Cu) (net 22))
 (segment (start 135.9334 87.3) (end 135.5 87.7334) (width 0.254) (layer F.Cu) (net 22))
 (segment (start 135.5 90.016) (end 136.7 91.216) (width 0.254) (layer F.Cu) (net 22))
 (segment (start 135.5 87.7334) (end 135.5 90.016) (width 0.254) (layer F.Cu) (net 22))
 (segment (start 128.165 110) (end 128.165 103.335) (width 0.254) (layer F.Cu) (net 8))
 (segment (start 121.835 92.335) (end 121.835 80) (width 0.254) (layer B.Cu) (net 8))
 (segment (start 130.5 101) (end 121.835 92.335) (width 0.254) (layer B.Cu) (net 8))
 (via (at 130.5 101) (size 0.889) (layers F.Cu B.Cu) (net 8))
 (segment (start 128.165 103.335) (end 130.5 101) (width 0.254) (layer F.Cu) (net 8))
 (segment (start 127.02 107.46) (end 127.02 103.18) (width 0.254) (layer F.Cu) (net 13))
 (segment (start 122.98 92.18) (end 122.98 82.54) (width 0.254) (layer B.Cu) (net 13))
 (segment (start 130.5 99.7) (end 122.98 92.18) (width 0.254) (layer B.Cu) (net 13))
 (via (at 130.5 99.7) (size 0.889) (layers F.Cu B.Cu) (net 13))
 (segment (start 127.02 103.18) (end 130.5 99.7) (width 0.254) (layer F.Cu) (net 13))
 (segment (start 124.73 107.46) (end 124.73 102.87) (width 0.254) (layer F.Cu) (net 14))
 (segment (start 125.27 91.87) (end 125.27 82.54) (width 0.254) (layer B.Cu) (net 14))
 (segment (start 130.5 97.1) (end 125.27 91.87) (width 0.254) (layer B.Cu) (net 14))
 (via (at 130.5 97.1) (size 0.889) (layers F.Cu B.Cu) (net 14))
 (segment (start 124.73 102.87) (end 130.5 97.1) (width 0.254) (layer F.Cu) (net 14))
 (segment (start 122.44 107.46) (end 122.44 102.56) (width 0.254) (layer F.Cu) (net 15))
 (segment (start 127.56 91.56) (end 127.56 82.54) (width 0.254) (layer B.Cu) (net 15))
 (segment (start 130.5 94.5) (end 127.56 91.56) (width 0.254) (layer B.Cu) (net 15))
 (via (at 130.5 94.5) (size 0.889) (layers F.Cu B.Cu) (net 15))
 (segment (start 122.44 102.56) (end 130.5 94.5) (width 0.254) (layer F.Cu) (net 15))
 (segment (start 130.455 110) (end 130.455 103.645) (width 0.254) (layer F.Cu) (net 7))
 (segment (start 119.545 92.645) (end 119.545 80) (width 0.254) (layer B.Cu) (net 7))
 (segment (start 130.5 103.6) (end 119.545 92.645) (width 0.254) (layer B.Cu) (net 7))
 (via (at 130.5 103.6) (size 0.889) (layers F.Cu B.Cu) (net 7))
 (segment (start 130.455 103.645) (end 130.5 103.6) (width 0.254) (layer F.Cu) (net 7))
 (segment (start 125.875 110) (end 125.875 103.025) (width 0.254) (layer F.Cu) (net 9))
 (segment (start 124.125 92.025) (end 124.125 80) (width 0.254) (layer B.Cu) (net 9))
 (segment (start 130.5 98.4) (end 124.125 92.025) (width 0.254) (layer B.Cu) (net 9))
 (via (at 130.5 98.4) (size 0.889) (layers F.Cu B.Cu) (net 9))
 (segment (start 125.875 103.025) (end 130.5 98.4) (width 0.254) (layer F.Cu) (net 9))
 (segment (start 119 94.8) (end 121.84 91.96) (width 0.254) (layer F.Cu) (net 16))
 (segment (start 128.17 103.97) (end 119 94.8) (width 0.254) (layer B.Cu) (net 16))
 (via (at 119 94.8) (size 0.889) (layers F.Cu B.Cu) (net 16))
 (segment (start 129.31 112.54) (end 129.31 109.31) (width 0.254) (layer B.Cu) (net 16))
 (segment (start 129.31 109.31) (end 128.17 108.17) (width 0.254) (layer B.Cu) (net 16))
 (segment (start 128.17 108.17) (end 128.17 103.97) (width 0.254) (layer B.Cu) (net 16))
 (segment (start 120.69 80.7) (end 120.69 77.46) (width 0.254) (layer F.Cu) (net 16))
 (segment (start 121.84 81.85) (end 120.69 80.7) (width 0.254) (layer F.Cu) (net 16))
 (segment (start 121.84 91.96) (end 121.84 81.85) (width 0.254) (layer F.Cu) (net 16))
 (segment (start 119 96.1) (end 124.13 90.97) (width 0.254) (layer F.Cu) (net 17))
 (segment (start 125.87 102.97) (end 119 96.1) (width 0.254) (layer B.Cu) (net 17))
 (via (at 119 96.1) (size 0.889) (layers F.Cu B.Cu) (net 17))
 (segment (start 127.02 112.54) (end 127.02 109.3) (width 0.254) (layer B.Cu) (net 17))
 (segment (start 127.02 109.3) (end 125.87 108.15) (width 0.254) (layer B.Cu) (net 17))
 (segment (start 125.87 108.15) (end 125.87 102.97) (width 0.254) (layer B.Cu) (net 17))
 (segment (start 122.98 80.72) (end 122.98 77.46) (width 0.254) (layer F.Cu) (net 17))
 (segment (start 124.13 81.87) (end 122.98 80.72) (width 0.254) (layer F.Cu) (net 17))
 (segment (start 124.13 90.97) (end 124.13 81.87) (width 0.254) (layer F.Cu) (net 17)))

